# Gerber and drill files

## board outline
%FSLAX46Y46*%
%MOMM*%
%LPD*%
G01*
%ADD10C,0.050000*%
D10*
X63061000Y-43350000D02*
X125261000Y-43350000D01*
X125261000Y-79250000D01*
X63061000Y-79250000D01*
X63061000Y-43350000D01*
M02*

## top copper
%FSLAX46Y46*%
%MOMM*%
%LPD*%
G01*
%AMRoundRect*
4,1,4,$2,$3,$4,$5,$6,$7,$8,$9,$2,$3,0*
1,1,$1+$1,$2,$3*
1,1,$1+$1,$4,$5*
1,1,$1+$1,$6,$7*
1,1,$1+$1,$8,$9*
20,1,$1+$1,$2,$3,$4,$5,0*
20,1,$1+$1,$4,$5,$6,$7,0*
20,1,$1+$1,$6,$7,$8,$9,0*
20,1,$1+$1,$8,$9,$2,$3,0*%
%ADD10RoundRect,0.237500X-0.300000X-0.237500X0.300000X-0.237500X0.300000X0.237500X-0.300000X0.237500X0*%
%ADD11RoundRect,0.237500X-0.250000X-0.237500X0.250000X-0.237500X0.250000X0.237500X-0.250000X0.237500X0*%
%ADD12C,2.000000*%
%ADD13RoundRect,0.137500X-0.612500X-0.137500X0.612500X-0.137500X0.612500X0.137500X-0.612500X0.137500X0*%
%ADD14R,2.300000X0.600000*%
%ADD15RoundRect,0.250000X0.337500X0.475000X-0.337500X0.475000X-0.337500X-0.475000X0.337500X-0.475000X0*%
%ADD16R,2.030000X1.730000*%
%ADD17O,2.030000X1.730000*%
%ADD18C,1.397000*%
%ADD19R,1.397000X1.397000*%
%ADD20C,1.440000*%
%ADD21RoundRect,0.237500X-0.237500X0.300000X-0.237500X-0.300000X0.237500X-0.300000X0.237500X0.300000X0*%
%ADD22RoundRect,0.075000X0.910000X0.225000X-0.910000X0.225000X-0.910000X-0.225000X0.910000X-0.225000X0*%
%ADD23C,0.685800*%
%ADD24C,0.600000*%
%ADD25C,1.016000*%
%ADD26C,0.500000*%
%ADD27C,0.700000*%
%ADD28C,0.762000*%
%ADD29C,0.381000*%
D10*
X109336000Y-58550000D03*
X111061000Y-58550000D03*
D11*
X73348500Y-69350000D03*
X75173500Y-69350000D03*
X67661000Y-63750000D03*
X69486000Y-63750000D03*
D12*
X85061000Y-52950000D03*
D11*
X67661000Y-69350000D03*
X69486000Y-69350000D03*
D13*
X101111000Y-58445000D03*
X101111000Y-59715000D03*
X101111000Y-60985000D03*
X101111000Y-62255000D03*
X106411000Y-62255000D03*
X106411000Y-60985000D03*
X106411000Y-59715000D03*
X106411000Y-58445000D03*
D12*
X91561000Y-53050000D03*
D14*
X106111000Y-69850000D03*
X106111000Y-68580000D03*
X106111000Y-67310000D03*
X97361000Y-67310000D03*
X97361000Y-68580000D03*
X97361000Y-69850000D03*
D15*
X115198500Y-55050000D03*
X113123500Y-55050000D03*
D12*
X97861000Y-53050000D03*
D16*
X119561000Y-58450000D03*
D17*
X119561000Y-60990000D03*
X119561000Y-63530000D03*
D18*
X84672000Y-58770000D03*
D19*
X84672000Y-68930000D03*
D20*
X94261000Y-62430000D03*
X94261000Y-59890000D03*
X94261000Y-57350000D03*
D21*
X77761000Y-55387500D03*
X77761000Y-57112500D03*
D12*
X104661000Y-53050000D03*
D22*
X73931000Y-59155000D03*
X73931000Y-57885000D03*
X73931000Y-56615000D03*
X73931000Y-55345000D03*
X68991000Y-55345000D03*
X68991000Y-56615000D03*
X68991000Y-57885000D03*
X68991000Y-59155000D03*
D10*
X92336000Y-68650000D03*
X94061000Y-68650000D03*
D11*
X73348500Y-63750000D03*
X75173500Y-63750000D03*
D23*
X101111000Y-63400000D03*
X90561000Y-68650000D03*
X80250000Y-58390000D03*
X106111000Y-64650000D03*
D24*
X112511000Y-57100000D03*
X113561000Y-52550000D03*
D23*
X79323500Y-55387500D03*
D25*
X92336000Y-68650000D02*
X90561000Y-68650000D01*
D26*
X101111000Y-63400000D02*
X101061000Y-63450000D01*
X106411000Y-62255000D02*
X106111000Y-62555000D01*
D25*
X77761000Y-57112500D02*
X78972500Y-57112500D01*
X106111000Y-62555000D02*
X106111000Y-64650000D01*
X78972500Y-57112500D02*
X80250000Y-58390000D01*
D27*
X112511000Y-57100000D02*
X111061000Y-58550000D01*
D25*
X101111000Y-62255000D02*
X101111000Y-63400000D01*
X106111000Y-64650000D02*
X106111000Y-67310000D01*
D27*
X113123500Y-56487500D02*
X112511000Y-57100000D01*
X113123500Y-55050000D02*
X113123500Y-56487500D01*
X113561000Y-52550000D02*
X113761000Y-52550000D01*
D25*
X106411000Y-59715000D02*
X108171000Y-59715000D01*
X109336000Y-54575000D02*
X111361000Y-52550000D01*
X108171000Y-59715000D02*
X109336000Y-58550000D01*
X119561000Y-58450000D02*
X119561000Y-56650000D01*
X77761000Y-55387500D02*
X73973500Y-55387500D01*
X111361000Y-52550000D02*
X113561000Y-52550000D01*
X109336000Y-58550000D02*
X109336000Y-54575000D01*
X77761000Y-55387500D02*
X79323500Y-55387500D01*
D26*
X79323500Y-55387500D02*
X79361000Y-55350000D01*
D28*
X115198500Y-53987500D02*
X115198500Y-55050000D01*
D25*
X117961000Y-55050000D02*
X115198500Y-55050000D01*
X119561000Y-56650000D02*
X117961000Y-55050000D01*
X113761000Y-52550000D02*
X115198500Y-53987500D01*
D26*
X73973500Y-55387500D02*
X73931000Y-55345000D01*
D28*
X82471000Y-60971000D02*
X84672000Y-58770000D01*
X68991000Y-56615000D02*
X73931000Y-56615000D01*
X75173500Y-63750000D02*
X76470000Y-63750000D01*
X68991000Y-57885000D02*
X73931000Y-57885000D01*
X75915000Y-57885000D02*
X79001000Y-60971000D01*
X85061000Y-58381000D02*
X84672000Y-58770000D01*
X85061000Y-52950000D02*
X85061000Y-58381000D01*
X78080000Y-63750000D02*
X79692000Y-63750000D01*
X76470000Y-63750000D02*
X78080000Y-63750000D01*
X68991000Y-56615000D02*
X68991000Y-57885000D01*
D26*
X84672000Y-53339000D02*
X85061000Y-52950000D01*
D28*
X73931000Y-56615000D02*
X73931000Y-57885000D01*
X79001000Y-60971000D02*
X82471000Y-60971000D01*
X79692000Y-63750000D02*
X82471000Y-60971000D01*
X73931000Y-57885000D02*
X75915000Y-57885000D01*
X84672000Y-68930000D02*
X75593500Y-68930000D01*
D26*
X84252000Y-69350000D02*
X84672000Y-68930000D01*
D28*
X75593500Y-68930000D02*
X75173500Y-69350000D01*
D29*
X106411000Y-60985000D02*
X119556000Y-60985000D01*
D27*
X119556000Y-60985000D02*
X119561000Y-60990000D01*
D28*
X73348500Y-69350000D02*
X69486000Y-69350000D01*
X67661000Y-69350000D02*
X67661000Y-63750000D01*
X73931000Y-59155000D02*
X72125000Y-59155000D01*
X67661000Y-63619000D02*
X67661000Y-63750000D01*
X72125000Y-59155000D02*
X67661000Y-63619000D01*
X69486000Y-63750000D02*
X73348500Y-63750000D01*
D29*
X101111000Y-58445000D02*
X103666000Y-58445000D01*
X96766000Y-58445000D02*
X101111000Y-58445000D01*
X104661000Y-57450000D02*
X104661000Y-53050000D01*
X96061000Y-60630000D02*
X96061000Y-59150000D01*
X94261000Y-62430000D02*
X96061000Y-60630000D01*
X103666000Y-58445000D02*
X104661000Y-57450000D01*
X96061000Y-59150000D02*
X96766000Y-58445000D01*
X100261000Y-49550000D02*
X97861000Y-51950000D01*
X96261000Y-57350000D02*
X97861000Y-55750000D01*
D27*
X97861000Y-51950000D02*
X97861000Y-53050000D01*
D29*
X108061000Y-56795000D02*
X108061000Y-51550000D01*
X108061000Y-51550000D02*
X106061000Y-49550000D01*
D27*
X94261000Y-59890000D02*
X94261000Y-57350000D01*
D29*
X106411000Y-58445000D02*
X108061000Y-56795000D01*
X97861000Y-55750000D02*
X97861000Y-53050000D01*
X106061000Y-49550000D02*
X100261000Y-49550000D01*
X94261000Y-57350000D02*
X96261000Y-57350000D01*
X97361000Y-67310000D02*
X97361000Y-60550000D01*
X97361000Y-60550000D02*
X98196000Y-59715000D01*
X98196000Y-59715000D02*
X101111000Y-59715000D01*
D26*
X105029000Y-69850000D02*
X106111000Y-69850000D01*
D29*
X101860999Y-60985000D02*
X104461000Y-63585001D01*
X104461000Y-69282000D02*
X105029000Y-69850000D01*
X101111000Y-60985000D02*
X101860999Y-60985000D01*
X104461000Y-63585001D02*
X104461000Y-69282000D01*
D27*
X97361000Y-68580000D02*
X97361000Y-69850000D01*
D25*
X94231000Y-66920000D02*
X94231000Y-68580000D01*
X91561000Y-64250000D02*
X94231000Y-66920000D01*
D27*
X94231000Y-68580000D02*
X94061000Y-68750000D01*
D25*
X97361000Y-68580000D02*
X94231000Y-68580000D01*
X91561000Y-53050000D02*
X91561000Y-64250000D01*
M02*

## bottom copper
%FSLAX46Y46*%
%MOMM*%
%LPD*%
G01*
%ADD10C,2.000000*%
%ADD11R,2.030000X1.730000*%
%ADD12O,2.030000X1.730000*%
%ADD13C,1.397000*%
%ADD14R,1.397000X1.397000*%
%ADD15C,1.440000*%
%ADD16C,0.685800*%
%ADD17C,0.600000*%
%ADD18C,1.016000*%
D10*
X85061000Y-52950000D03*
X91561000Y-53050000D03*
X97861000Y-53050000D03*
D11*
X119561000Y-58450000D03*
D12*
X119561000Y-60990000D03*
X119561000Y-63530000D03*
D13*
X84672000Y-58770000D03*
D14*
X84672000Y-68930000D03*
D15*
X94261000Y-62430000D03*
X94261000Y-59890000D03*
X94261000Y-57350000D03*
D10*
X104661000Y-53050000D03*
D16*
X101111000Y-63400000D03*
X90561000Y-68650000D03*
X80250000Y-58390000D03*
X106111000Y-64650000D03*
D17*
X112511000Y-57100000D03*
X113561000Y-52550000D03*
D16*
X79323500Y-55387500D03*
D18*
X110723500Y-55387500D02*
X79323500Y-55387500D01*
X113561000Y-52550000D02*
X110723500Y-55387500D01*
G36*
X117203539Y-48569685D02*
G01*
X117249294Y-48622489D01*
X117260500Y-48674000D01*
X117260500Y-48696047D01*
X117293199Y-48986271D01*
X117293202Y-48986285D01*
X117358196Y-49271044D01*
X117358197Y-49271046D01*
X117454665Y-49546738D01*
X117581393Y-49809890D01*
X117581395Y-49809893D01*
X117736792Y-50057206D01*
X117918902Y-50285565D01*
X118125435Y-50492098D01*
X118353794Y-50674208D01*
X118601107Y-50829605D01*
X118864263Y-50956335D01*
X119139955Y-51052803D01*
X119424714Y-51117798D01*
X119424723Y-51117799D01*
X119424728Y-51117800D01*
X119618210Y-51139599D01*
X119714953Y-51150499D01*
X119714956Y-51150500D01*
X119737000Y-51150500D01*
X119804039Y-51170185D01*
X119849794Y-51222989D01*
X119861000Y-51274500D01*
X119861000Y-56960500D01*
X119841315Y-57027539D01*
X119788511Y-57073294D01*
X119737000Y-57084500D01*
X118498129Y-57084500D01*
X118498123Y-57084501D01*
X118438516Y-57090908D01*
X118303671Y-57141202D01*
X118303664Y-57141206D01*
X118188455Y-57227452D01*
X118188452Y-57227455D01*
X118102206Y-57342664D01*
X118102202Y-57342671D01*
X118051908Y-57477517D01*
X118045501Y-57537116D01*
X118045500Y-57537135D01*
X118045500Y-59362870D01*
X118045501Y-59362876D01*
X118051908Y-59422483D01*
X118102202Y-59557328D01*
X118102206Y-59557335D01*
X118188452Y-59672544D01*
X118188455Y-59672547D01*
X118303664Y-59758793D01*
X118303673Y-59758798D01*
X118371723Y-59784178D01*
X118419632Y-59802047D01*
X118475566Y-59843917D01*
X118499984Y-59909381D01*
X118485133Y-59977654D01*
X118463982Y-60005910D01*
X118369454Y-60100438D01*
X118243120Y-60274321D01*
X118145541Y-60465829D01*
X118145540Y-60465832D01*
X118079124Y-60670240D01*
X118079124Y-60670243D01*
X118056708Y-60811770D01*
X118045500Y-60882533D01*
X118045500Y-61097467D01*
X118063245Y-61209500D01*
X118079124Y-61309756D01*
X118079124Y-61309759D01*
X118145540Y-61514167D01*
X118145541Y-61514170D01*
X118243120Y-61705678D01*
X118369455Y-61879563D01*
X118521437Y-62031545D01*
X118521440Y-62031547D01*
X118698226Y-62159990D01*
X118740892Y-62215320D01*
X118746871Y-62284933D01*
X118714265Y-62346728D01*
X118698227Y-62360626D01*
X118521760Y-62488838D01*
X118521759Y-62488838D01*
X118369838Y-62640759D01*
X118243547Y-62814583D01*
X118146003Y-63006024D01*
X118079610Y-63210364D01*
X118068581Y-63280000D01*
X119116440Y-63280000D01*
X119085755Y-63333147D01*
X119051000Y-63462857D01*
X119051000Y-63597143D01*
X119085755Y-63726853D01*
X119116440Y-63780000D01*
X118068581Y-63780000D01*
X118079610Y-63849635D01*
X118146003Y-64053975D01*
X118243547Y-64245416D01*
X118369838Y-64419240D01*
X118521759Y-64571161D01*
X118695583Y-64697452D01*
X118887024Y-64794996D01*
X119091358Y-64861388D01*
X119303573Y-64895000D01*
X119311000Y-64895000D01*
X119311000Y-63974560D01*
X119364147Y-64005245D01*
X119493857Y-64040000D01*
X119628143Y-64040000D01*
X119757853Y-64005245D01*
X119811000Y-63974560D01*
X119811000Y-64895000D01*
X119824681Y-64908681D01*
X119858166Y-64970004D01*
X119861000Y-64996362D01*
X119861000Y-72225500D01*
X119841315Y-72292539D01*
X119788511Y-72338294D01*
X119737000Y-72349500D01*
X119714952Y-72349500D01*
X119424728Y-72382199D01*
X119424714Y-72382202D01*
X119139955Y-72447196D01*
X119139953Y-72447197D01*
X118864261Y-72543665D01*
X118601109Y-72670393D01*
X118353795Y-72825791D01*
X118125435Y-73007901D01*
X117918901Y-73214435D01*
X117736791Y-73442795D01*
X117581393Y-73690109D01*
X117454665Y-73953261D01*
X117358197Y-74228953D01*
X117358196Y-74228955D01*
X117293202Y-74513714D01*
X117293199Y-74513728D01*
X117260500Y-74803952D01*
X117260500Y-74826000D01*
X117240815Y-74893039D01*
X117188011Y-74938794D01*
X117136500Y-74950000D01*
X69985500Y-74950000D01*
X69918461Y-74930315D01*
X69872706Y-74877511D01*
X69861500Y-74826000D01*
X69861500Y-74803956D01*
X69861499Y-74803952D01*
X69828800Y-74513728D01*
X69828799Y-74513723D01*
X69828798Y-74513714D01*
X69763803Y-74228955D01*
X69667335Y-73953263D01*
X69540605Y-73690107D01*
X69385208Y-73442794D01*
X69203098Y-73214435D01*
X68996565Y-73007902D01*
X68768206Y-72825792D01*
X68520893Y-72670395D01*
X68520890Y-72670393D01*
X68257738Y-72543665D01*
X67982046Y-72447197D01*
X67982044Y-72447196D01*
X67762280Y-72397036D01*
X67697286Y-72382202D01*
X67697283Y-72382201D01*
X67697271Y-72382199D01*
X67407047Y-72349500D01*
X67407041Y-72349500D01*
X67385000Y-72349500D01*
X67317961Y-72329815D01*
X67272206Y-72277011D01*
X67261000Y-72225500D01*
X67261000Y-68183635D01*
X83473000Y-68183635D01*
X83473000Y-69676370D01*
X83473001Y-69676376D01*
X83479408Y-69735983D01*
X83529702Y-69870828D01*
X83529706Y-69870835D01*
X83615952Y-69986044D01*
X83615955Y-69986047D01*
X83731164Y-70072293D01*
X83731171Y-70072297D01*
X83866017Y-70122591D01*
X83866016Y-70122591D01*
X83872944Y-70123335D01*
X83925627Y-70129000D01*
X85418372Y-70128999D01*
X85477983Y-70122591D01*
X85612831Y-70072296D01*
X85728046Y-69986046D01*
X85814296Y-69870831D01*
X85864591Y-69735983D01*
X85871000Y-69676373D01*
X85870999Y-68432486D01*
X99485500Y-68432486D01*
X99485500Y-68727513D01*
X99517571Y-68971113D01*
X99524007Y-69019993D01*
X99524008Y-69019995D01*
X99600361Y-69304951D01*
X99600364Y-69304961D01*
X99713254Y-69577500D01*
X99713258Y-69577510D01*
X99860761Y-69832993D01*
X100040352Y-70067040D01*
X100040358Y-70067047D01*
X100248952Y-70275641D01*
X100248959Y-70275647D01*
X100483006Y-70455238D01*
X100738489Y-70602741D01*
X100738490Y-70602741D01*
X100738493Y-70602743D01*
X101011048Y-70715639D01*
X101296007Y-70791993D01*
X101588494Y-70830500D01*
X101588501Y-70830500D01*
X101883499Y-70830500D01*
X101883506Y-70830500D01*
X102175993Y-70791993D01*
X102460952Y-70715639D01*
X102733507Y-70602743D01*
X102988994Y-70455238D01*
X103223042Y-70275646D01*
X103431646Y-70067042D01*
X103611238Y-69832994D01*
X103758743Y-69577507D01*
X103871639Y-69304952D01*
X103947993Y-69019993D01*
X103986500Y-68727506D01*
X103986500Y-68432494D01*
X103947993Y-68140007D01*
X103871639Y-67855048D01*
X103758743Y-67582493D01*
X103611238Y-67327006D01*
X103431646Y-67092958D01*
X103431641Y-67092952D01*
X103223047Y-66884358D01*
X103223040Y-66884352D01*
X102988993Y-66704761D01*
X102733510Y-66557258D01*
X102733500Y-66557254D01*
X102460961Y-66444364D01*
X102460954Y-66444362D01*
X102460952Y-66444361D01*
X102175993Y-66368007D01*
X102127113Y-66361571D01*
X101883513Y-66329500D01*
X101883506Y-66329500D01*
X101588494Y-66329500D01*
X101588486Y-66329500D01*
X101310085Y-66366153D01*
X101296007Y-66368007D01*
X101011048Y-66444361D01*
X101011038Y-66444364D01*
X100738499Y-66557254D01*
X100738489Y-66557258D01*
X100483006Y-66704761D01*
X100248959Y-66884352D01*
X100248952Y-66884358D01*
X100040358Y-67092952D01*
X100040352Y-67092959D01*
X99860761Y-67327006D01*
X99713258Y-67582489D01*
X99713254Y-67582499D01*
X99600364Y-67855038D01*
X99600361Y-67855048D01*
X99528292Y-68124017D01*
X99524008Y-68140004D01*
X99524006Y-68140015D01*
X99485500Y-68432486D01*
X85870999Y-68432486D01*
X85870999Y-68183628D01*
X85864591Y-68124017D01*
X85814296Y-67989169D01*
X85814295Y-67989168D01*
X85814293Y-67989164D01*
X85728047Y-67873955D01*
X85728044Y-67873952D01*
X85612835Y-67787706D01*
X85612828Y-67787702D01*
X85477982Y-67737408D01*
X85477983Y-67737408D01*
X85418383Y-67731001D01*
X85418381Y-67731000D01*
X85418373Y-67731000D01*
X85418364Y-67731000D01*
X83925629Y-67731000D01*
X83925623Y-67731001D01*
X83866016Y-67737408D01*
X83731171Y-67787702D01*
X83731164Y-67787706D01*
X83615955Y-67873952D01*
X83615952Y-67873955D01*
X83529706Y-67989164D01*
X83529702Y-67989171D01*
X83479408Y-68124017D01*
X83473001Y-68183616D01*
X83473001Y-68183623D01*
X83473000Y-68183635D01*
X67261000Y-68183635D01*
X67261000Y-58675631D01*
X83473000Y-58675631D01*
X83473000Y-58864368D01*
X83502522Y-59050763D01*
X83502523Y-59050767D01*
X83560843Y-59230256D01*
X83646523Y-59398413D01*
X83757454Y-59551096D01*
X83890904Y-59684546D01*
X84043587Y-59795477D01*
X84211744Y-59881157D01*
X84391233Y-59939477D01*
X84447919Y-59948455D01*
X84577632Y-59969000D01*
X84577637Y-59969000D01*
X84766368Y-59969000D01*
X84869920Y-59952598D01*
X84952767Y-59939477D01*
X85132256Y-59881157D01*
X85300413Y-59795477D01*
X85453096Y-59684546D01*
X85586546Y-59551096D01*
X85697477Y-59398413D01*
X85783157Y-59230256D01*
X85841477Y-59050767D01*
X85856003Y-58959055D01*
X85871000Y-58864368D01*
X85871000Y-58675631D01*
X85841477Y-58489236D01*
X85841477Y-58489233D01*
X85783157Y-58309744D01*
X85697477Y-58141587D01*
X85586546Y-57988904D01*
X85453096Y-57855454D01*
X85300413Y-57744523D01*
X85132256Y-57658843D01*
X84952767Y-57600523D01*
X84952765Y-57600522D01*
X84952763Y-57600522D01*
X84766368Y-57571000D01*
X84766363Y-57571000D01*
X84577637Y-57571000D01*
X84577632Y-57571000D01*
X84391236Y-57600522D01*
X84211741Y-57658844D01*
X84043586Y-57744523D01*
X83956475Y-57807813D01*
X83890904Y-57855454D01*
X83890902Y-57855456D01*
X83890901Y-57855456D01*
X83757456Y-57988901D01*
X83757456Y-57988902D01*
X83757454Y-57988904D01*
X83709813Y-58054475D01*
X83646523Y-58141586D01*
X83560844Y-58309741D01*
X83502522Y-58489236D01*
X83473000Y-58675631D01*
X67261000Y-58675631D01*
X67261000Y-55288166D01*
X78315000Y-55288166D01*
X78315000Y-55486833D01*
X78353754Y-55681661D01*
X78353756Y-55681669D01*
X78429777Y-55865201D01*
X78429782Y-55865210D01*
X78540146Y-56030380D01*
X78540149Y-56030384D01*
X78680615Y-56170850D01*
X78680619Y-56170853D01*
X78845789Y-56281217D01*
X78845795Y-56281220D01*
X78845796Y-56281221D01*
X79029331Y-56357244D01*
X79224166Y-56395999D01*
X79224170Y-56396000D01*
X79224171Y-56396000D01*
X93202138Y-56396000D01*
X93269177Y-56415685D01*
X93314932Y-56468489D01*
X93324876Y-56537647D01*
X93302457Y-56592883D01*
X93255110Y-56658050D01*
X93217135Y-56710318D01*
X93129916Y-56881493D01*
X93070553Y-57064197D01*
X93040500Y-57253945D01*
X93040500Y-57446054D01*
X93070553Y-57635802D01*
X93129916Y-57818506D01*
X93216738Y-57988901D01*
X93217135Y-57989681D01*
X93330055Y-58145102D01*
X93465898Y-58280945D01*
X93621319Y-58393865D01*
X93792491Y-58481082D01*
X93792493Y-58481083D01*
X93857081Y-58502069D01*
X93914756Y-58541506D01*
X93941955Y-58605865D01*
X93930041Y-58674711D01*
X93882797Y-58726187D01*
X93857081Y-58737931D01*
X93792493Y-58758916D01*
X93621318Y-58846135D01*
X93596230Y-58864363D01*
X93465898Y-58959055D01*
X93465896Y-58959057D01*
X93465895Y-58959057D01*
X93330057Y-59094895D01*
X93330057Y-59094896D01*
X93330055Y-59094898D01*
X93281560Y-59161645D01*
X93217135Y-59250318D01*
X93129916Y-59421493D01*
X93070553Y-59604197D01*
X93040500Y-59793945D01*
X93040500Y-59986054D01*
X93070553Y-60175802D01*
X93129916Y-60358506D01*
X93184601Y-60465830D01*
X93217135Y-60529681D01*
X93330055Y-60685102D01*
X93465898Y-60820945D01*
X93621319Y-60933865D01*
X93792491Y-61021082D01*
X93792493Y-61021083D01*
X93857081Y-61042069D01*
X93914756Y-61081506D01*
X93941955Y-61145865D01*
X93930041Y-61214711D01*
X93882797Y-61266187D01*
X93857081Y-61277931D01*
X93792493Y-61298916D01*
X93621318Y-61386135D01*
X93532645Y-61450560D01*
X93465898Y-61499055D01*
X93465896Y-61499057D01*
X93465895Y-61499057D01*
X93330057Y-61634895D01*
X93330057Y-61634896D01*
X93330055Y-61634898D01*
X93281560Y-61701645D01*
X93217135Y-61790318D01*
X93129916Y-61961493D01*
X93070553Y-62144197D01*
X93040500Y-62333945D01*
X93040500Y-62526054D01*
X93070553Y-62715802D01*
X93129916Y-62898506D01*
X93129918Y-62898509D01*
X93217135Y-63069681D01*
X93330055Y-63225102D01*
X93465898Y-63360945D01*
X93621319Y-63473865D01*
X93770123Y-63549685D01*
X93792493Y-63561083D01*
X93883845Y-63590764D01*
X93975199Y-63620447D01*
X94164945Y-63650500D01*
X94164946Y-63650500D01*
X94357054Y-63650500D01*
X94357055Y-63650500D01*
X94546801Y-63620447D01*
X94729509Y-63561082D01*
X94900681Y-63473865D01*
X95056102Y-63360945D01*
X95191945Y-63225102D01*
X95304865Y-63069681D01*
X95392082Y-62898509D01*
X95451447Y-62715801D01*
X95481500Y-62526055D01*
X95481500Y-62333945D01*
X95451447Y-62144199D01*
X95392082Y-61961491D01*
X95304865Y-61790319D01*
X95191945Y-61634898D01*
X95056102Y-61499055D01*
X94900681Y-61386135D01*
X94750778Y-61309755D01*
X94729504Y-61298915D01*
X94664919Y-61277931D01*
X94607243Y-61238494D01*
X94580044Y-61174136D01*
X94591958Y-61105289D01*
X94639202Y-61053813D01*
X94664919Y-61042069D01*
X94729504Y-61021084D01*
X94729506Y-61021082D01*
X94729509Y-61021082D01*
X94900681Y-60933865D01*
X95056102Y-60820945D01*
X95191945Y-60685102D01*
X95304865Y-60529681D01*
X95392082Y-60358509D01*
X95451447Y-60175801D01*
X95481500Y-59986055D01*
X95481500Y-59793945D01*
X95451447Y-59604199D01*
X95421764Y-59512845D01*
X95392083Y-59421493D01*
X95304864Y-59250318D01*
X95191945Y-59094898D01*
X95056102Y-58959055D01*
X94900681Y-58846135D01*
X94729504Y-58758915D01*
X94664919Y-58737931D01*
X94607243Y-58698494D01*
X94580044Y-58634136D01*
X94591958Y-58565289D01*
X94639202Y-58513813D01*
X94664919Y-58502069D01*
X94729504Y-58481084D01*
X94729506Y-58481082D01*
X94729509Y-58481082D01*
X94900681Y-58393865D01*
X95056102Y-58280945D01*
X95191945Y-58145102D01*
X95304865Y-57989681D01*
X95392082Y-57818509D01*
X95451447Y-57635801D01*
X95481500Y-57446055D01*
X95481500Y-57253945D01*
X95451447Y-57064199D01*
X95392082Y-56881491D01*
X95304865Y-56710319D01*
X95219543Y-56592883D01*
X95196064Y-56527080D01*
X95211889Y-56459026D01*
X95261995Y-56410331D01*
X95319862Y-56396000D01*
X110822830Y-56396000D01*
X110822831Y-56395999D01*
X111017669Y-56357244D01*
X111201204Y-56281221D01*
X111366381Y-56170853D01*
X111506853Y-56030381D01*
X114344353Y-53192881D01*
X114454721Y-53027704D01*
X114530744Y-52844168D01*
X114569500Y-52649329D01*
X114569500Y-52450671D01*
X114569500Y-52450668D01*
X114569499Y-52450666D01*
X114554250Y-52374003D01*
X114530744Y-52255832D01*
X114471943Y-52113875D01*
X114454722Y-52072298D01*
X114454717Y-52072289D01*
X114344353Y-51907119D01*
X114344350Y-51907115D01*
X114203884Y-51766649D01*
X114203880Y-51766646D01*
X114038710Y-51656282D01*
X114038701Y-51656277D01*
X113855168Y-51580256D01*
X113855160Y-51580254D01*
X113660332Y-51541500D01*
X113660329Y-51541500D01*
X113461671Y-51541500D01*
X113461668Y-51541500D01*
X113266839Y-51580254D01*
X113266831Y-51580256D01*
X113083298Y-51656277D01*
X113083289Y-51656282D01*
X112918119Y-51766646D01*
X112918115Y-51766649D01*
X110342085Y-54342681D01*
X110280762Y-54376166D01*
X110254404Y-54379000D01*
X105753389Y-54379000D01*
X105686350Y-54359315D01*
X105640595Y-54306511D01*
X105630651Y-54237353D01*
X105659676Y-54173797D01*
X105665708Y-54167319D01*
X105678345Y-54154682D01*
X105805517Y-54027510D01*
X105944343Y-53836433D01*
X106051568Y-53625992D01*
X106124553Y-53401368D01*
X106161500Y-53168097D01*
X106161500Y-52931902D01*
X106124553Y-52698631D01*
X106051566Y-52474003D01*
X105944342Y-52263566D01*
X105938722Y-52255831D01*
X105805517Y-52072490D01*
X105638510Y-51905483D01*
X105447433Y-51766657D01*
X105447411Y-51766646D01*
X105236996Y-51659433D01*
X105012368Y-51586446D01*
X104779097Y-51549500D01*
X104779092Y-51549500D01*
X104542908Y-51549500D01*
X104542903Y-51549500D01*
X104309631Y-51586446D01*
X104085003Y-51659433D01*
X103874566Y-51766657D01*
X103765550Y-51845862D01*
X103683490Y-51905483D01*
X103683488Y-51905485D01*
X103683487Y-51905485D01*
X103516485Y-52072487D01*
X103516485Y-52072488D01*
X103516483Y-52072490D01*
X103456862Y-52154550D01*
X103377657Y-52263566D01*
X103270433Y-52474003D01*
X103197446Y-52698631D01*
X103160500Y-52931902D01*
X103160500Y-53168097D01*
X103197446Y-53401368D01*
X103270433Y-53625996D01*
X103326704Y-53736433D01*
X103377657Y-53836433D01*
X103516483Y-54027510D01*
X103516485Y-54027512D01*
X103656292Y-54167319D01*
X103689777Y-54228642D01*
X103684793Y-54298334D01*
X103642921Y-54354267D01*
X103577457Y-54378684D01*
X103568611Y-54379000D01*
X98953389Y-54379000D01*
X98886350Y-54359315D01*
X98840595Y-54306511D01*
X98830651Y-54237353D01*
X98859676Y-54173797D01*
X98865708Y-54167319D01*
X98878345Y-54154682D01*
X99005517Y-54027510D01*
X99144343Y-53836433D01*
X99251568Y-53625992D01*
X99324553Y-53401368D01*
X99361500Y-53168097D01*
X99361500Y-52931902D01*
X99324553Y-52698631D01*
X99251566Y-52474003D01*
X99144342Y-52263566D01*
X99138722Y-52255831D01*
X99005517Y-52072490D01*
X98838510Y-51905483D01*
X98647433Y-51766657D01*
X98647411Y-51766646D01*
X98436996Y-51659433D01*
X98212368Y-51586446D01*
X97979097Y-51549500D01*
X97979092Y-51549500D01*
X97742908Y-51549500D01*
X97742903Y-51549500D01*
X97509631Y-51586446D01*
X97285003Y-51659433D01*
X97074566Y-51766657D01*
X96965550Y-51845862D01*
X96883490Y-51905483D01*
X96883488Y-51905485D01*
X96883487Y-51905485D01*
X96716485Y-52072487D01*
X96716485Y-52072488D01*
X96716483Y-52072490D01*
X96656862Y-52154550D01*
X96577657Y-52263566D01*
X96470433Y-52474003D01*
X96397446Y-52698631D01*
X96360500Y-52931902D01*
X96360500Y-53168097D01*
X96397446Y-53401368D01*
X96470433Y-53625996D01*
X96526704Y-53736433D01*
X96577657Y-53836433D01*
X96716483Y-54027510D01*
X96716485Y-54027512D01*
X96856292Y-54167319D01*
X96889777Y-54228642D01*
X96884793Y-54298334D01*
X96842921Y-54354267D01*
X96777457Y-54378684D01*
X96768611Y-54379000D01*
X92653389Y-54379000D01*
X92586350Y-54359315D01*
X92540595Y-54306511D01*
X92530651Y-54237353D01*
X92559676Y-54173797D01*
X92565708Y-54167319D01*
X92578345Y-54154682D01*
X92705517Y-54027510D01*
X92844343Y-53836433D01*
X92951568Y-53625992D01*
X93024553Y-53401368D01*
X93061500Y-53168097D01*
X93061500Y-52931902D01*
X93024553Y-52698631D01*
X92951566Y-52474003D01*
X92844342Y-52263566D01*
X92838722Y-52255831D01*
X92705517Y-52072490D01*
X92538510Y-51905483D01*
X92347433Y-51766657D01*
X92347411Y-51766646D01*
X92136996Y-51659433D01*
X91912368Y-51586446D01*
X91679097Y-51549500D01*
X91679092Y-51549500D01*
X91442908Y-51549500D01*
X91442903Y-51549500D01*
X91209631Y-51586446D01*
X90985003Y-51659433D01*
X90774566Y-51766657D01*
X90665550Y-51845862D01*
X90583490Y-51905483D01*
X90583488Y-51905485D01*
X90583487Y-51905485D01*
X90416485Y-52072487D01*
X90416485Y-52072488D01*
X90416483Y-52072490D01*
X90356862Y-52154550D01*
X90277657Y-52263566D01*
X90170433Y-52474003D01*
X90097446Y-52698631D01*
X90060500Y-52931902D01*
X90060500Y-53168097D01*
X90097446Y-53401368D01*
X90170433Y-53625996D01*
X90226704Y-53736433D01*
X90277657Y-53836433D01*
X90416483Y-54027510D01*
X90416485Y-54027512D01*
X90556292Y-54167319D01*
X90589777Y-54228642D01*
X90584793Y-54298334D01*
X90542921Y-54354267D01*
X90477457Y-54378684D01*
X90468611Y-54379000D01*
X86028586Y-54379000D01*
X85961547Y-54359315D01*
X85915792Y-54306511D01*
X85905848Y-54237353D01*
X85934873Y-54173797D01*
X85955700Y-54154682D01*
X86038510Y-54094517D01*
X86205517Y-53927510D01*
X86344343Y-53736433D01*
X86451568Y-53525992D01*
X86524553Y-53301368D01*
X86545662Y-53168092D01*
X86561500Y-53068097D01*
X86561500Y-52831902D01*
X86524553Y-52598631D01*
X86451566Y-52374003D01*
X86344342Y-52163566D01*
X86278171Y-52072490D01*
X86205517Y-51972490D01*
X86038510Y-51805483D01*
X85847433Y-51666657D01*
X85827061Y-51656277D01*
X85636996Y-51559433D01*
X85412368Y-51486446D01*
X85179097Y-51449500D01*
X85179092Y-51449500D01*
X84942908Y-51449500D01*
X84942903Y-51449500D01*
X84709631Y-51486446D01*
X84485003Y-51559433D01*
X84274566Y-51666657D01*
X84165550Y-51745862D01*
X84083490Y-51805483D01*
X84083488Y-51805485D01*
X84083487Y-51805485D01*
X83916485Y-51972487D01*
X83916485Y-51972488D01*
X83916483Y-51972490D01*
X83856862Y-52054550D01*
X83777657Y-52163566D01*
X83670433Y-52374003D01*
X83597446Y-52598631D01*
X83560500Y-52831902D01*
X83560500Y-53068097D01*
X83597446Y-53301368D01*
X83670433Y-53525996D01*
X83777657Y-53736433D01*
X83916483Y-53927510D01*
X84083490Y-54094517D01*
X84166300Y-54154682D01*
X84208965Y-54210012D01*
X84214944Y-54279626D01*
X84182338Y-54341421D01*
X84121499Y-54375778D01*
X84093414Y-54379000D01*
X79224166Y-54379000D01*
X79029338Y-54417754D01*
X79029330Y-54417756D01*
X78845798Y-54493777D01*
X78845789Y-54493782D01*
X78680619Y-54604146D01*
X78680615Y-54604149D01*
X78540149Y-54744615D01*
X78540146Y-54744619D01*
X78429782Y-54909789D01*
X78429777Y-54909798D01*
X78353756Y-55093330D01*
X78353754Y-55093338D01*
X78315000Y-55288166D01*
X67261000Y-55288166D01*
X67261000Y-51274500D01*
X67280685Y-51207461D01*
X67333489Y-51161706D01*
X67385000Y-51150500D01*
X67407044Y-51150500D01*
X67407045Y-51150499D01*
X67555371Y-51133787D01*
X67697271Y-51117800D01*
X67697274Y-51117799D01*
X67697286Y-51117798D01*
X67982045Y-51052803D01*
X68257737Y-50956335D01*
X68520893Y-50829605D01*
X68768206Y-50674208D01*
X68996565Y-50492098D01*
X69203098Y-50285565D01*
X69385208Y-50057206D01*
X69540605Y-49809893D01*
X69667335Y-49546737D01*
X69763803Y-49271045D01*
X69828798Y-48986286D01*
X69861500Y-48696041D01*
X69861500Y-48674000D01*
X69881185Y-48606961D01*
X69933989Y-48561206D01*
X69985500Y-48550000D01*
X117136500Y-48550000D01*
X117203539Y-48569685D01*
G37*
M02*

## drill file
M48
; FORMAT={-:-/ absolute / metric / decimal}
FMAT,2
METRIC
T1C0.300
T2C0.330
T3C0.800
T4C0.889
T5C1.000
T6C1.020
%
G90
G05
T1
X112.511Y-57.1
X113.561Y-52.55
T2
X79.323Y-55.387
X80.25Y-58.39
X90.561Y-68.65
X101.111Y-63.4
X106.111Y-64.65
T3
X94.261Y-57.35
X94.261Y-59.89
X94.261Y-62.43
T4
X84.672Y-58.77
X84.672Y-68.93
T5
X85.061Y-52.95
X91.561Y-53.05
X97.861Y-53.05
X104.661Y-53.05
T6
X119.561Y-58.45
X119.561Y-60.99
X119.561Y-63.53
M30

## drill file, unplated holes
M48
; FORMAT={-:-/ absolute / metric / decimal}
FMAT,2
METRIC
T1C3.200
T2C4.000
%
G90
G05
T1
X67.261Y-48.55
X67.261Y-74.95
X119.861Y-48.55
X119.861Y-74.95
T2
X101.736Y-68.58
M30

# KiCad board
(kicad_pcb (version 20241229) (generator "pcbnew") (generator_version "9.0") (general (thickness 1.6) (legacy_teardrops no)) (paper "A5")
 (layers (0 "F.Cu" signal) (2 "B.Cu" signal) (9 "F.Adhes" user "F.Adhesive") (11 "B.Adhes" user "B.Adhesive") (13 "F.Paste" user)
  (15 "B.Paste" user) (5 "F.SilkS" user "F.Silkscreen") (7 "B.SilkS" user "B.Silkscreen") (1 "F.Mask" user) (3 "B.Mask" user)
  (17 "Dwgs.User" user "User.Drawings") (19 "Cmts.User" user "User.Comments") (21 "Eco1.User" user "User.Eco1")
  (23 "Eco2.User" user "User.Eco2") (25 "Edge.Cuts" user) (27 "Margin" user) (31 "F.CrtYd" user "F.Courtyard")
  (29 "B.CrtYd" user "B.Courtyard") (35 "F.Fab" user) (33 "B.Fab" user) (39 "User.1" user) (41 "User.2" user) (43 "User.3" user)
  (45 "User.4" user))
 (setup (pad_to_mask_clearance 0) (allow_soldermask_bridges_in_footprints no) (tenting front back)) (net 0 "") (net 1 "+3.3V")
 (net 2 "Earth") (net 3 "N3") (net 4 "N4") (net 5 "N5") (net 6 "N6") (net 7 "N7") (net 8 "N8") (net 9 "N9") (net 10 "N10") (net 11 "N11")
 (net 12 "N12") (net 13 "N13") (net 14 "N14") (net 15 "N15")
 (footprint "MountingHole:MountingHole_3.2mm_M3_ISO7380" (layer "F.Cu") (at 67.261 48.55)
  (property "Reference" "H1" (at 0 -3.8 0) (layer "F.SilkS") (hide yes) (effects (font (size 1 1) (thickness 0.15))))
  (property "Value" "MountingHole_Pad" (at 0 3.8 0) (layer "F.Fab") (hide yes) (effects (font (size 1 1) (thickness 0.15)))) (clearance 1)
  (pad "" np_thru_hole circle (at 0 0) (size 3.2 3.2) (drill 3.2) (layers "*.Cu" "*.Mask")))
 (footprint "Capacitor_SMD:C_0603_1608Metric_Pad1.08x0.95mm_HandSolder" (layer "F.Cu") (at 110.1985 58.55)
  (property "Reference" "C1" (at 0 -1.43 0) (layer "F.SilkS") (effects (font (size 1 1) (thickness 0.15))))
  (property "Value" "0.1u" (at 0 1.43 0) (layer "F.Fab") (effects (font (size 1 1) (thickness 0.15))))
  (pad "1" smd roundrect (at -0.8625 0) (size 1.075 0.95) (layers "F.Cu" "F.Mask" "F.Paste") (roundrect_rratio 0.25) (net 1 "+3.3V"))
  (pad "2" smd roundrect (at 0.8625 0) (size 1.075 0.95) (layers "F.Cu" "F.Mask" "F.Paste") (roundrect_rratio 0.25) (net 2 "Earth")))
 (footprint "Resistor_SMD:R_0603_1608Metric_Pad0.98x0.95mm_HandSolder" (layer "F.Cu") (at 74.261 69.35)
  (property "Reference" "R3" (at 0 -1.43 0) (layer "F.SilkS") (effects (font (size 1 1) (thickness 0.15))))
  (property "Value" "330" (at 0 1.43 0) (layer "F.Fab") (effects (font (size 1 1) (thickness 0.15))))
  (pad "1" smd roundrect (at -0.9125 0) (size 0.975 0.95) (layers "F.Cu" "F.Mask" "F.Paste") (roundrect_rratio 0.25) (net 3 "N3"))
  (pad "2" smd roundrect (at 0.9125 0) (size 0.975 0.95) (layers "F.Cu" "F.Mask" "F.Paste") (roundrect_rratio 0.25) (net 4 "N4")))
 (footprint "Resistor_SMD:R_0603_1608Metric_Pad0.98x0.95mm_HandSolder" (layer "F.Cu") (at 68.5735 63.75)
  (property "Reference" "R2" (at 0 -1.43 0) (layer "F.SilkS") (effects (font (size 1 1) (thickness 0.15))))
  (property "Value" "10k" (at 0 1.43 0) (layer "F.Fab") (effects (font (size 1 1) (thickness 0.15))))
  (pad "1" smd roundrect (at -0.9125 0) (size 0.975 0.95) (layers "F.Cu" "F.Mask" "F.Paste") (roundrect_rratio 0.25) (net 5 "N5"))
  (pad "2" smd roundrect (at 0.9125 0) (size 0.975 0.95) (layers "F.Cu" "F.Mask" "F.Paste") (roundrect_rratio 0.25) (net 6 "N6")))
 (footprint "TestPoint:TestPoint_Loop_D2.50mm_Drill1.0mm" (layer "F.Cu") (at 85.061 52.95 180)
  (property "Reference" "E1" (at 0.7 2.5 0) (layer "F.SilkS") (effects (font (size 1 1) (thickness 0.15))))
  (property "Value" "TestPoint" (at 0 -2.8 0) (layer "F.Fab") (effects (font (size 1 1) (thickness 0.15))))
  (pad "1" thru_hole circle (at 0 0 180) (size 2 2) (drill 1) (layers "*.Cu" "*.Mask") (remove_unused_layers no) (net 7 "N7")))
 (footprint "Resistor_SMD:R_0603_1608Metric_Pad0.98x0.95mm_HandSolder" (layer "F.Cu") (at 68.5735 69.35)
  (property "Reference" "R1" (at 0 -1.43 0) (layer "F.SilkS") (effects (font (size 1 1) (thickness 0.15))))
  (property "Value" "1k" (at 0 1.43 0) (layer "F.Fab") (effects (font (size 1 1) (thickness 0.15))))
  (pad "1" smd roundrect (at -0.9125 0) (size 0.975 0.95) (layers "F.Cu" "F.Mask" "F.Paste") (roundrect_rratio 0.25) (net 5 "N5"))
  (pad "2" smd roundrect (at 0.9125 0) (size 0.975 0.95) (layers "F.Cu" "F.Mask" "F.Paste") (roundrect_rratio 0.25) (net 3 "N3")))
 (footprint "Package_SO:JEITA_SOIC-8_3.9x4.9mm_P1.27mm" (layer "F.Cu") (at 103.761 60.35)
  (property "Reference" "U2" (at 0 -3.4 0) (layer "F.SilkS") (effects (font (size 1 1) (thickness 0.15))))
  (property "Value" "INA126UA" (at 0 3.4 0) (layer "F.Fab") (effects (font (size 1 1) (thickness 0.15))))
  (pad "1" smd roundrect (at -2.65 -1.905) (size 1.5 0.55) (layers "F.Cu" "F.Mask" "F.Paste") (roundrect_rratio 0.25) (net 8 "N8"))
  (pad "2" smd roundrect (at -2.65 -0.635) (size 1.5 0.55) (layers "F.Cu" "F.Mask" "F.Paste") (roundrect_rratio 0.25) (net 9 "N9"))
  (pad "3" smd roundrect (at -2.65 0.635) (size 1.5 0.55) (layers "F.Cu" "F.Mask" "F.Paste") (roundrect_rratio 0.25) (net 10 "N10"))
  (pad "4" smd roundrect (at -2.65 1.905) (size 1.5 0.55) (layers "F.Cu" "F.Mask" "F.Paste") (roundrect_rratio 0.25) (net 2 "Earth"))
  (pad "5" smd roundrect (at 2.65 1.905) (size 1.5 0.55) (layers "F.Cu" "F.Mask" "F.Paste") (roundrect_rratio 0.25) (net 2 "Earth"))
  (pad "6" smd roundrect (at 2.65 0.635) (size 1.5 0.55) (layers "F.Cu" "F.Mask" "F.Paste") (roundrect_rratio 0.25) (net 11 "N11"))
  (pad "7" smd roundrect (at 2.65 -0.635) (size 1.5 0.55) (layers "F.Cu" "F.Mask" "F.Paste") (roundrect_rratio 0.25) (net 1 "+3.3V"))
  (pad "8" smd roundrect (at 2.65 -1.905) (size 1.5 0.55) (layers "F.Cu" "F.Mask" "F.Paste") (roundrect_rratio 0.25) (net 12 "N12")))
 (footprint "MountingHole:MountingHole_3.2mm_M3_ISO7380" (layer "F.Cu") (at 119.861 48.55)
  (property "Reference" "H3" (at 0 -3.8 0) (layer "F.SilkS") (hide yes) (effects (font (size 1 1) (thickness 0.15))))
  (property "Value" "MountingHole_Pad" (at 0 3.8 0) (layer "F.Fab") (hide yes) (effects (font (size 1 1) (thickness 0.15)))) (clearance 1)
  (pad "" np_thru_hole circle (at 0 0) (size 3.2 3.2) (drill 3.2) (layers "*.Cu" "*.Mask")))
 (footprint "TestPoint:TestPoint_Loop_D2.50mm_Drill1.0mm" (layer "F.Cu") (at 91.561 53.05 180)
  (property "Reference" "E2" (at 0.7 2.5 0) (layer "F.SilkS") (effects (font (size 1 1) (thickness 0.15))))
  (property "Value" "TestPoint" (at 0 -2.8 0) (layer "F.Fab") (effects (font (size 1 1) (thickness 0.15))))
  (pad "1" thru_hole circle (at 0 0 180) (size 2 2) (drill 1) (layers "*.Cu" "*.Mask") (remove_unused_layers no) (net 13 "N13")))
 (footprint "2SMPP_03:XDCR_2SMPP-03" (layer "F.Cu") (at 101.736 68.58 180)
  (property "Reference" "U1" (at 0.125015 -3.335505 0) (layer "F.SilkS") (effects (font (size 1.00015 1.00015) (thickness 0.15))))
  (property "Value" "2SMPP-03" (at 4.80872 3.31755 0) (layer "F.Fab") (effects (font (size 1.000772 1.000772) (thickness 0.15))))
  (pad "" np_thru_hole circle (at 0 0 180) (size 4 4) (drill 4) (layers "*.Cu" "*.Mask") (clearance 0.05))
  (pad "1" smd rect (at -4.375 -1.27 180) (size 2.3 0.6) (layers "F.Cu" "F.Mask" "F.Paste") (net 10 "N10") (solder_mask_margin 0.102))
  (pad "2" smd rect (at -4.375 0 180) (size 2.3 0.6) (layers "F.Cu" "F.Mask" "F.Paste") (solder_mask_margin 0.102))
  (pad "3" smd rect (at -4.375 1.27 180) (size 2.3 0.6) (layers "F.Cu" "F.Mask" "F.Paste") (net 2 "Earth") (solder_mask_margin 0.102))
  (pad "4" smd rect (at 4.375 1.27 180) (size 2.3 0.6) (layers "F.Cu" "F.Mask" "F.Paste") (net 9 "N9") (solder_mask_margin 0.102))
  (pad "5" smd rect (at 4.375 0 180) (size 2.3 0.6) (layers "F.Cu" "F.Mask" "F.Paste") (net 13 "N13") (solder_mask_margin 0.102))
  (pad "6" smd rect (at 4.375 -1.27 180) (size 2.3 0.6) (layers "F.Cu" "F.Mask" "F.Paste") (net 13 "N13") (solder_mask_margin 0.102)))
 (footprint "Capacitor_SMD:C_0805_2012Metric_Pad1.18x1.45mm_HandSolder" (layer "F.Cu") (at 114.161 55.05 180)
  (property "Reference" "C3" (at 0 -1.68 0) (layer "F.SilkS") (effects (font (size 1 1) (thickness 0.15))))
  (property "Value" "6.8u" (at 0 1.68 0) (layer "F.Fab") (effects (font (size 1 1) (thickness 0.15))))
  (pad "1" smd roundrect (at -1.0375 0 180) (size 1.175 1.45) (layers "F.Cu" "F.Mask" "F.Paste") (roundrect_rratio 0.212766) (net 1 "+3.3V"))
  (pad "2" smd roundrect (at 1.0375 0 180) (size 1.175 1.45) (layers "F.Cu" "F.Mask" "F.Paste") (roundrect_rratio 0.212766) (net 2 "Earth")))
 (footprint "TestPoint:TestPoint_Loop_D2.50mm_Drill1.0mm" (layer "F.Cu") (at 97.861 53.05 180)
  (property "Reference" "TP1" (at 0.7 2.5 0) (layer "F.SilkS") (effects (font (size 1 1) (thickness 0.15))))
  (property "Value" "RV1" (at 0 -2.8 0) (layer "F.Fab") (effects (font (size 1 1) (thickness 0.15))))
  (pad "1" thru_hole circle (at 0 0 180) (size 2 2) (drill 1) (layers "*.Cu" "*.Mask") (remove_unused_layers no) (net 12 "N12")))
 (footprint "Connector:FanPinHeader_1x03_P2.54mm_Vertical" (layer "F.Cu") (at 119.561 58.45 -90)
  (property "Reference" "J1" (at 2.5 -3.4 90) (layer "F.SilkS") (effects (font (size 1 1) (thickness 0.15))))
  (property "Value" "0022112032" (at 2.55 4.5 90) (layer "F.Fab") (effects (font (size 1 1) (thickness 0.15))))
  (pad "1" thru_hole rect (at 0 0) (size 2.03 1.73) (drill 1.02) (layers "*.Cu" "*.Mask") (remove_unused_layers no) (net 1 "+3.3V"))
  (pad "2" thru_hole oval (at 2.54 0) (size 2.03 1.73) (drill 1.02) (layers "*.Cu" "*.Mask") (remove_unused_layers no) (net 11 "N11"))
  (pad "3" thru_hole oval (at 5.08 0) (size 2.03 1.73) (drill 1.02) (layers "*.Cu" "*.Mask") (remove_unused_layers no) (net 2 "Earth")))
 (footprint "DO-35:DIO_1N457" (layer "F.Cu") (at 84.672 68.93 -90)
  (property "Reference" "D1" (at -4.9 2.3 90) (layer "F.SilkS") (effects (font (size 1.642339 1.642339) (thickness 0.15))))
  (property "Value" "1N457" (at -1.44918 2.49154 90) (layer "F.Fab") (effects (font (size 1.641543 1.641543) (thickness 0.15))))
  (pad "1" thru_hole circle (at -10.16 0 270) (size 1.397 1.397) (drill 0.889) (layers "*.Cu" "*.Mask") (remove_unused_layers no)
   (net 7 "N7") (solder_mask_margin 0.102))
  (pad "2" thru_hole rect (at 0 0 270) (size 1.397 1.397) (drill 0.889) (layers "*.Cu" "*.Mask") (remove_unused_layers no) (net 4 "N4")
   (solder_mask_margin 0.102)))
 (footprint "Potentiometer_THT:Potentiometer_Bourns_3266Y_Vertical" (layer "F.Cu") (at 94.261 62.43 -90)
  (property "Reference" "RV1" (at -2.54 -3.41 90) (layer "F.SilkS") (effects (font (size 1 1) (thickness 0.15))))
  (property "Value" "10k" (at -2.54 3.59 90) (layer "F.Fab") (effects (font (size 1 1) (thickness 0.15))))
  (pad "1" thru_hole circle (at 0 0 270) (size 1.44 1.44) (drill 0.8) (layers "*.Cu" "*.Mask") (remove_unused_layers no) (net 8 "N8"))
  (pad "2" thru_hole circle (at -2.54 0 270) (size 1.44 1.44) (drill 0.8) (layers "*.Cu" "*.Mask") (remove_unused_layers no) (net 12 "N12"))
  (pad "3" thru_hole circle (at -5.08 0 270) (size 1.44 1.44) (drill 0.8) (layers "*.Cu" "*.Mask") (remove_unused_layers no) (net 12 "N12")))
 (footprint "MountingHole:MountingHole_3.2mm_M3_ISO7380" (layer "F.Cu") (at 67.261 74.95)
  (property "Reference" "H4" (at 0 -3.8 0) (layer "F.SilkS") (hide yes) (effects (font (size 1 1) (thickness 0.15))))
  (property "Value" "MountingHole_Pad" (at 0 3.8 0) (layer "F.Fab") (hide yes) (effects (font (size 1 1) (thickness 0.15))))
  (pad "" np_thru_hole circle (at 0 0) (size 3.2 3.2) (drill 3.2) (layers "*.Cu" "*.Mask") (clearance 1)))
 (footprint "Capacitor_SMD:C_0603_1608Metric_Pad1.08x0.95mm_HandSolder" (layer "F.Cu") (at 77.761 56.25 -90)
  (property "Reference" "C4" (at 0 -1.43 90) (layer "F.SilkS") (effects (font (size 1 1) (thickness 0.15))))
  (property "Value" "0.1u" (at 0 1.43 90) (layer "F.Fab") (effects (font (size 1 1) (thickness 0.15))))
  (pad "1" smd roundrect (at -0.8625 0 270) (size 1.075 0.95) (layers "F.Cu" "F.Mask" "F.Paste") (roundrect_rratio 0.25) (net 1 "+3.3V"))
  (pad "2" smd roundrect (at 0.8625 0 270) (size 1.075 0.95) (layers "F.Cu" "F.Mask" "F.Paste") (roundrect_rratio 0.25) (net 2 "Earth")))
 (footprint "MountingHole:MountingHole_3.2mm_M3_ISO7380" (layer "F.Cu") (at 119.861 74.95)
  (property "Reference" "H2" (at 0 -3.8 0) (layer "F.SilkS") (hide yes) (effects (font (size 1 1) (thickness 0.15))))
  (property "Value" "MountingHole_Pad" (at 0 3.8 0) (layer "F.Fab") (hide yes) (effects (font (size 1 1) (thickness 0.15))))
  (pad "" np_thru_hole circle (at 0 0) (size 3.2 3.2) (drill 3.2) (layers "*.Cu" "*.Mask") (clearance 1)))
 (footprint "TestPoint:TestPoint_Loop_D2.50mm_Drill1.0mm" (layer "F.Cu") (at 104.661 53.05 180)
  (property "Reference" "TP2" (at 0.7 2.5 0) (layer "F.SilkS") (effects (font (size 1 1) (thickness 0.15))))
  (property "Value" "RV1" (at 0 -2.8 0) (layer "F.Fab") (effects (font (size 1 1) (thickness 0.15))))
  (pad "1" thru_hole circle (at 0 0 180) (size 2 2) (drill 1) (layers "*.Cu" "*.Mask") (remove_unused_layers no) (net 8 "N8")))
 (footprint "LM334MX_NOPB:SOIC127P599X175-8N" (layer "F.Cu") (at 71.461 57.25 180)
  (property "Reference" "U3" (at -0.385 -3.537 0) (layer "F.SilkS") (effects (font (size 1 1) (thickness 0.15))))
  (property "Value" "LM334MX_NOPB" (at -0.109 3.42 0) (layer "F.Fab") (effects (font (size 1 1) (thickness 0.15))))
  (pad "1" smd roundrect (at -2.47 -1.905 180) (size 1.97 0.6) (layers "F.Cu" "F.Mask" "F.Paste") (roundrect_rratio 0.125) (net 5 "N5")
   (solder_mask_margin 0.102))
  (pad "2" smd roundrect (at -2.47 -0.635 180) (size 1.97 0.6) (layers "F.Cu" "F.Mask" "F.Paste") (roundrect_rratio 0.125) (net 7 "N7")
   (solder_mask_margin 0.102))
  (pad "3" smd roundrect (at -2.47 0.635 180) (size 1.97 0.6) (layers "F.Cu" "F.Mask" "F.Paste") (roundrect_rratio 0.125) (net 7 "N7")
   (solder_mask_margin 0.102))
  (pad "4" smd roundrect (at -2.47 1.905 180) (size 1.97 0.6) (layers "F.Cu" "F.Mask" "F.Paste") (roundrect_rratio 0.125) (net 1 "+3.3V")
   (solder_mask_margin 0.102))
  (pad "5" smd roundrect (at 2.47 1.905 180) (size 1.97 0.6) (layers "F.Cu" "F.Mask" "F.Paste") (roundrect_rratio 0.125) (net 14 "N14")
   (solder_mask_margin 0.102))
  (pad "6" smd roundrect (at 2.47 0.635 180) (size 1.97 0.6) (layers "F.Cu" "F.Mask" "F.Paste") (roundrect_rratio 0.125) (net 7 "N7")
   (solder_mask_margin 0.102))
  (pad "7" smd roundrect (at 2.47 -0.635 180) (size 1.97 0.6) (layers "F.Cu" "F.Mask" "F.Paste") (roundrect_rratio 0.125) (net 7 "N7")
   (solder_mask_margin 0.102))
  (pad "8" smd roundrect (at 2.47 -1.905 180) (size 1.97 0.6) (layers "F.Cu" "F.Mask" "F.Paste") (roundrect_rratio 0.125) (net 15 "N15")
   (solder_mask_margin 0.102)))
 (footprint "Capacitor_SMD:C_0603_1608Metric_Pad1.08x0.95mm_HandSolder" (layer "F.Cu") (at 93.1985 68.65)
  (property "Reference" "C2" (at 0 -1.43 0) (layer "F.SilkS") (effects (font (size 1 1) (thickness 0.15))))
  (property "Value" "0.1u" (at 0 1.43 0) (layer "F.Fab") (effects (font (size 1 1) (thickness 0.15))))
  (pad "1" smd roundrect (at -0.8625 0) (size 1.075 0.95) (layers "F.Cu" "F.Mask" "F.Paste") (roundrect_rratio 0.25) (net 2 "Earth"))
  (pad "2" smd roundrect (at 0.8625 0) (size 1.075 0.95) (layers "F.Cu" "F.Mask" "F.Paste") (roundrect_rratio 0.25) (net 13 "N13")))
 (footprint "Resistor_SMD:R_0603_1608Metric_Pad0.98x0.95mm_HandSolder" (layer "F.Cu") (at 74.261 63.75)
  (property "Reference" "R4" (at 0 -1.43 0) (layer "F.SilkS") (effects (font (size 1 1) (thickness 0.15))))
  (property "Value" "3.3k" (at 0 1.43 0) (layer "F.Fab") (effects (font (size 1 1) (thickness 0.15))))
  (pad "1" smd roundrect (at -0.9125 0) (size 0.975 0.95) (layers "F.Cu" "F.Mask" "F.Paste") (roundrect_rratio 0.25) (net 6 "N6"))
  (pad "2" smd roundrect (at 0.9125 0) (size 0.975 0.95) (layers "F.Cu" "F.Mask" "F.Paste") (roundrect_rratio 0.25) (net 7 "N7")))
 (gr_rect (start 63.061 43.35) (end 125.261 79.25) (stroke (width 0.05) (type default)) (fill no) (layer "Edge.Cuts"))
 (segment (start 92.336 68.65) (end 90.561 68.65) (width 1.016) (layer "F.Cu") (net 2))
 (segment (start 101.111 63.4) (end 101.061 63.45) (width 0.5) (layer "F.Cu") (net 2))
 (segment (start 106.411 62.255) (end 106.111 62.555) (width 0.5) (layer "F.Cu") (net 2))
 (segment (start 77.761 57.1125) (end 78.9725 57.1125) (width 1.016) (layer "F.Cu") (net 2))
 (segment (start 106.111 62.555) (end 106.111 64.65) (width 1.016) (layer "F.Cu") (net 2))
 (segment (start 78.9725 57.1125) (end 80.25 58.39) (width 1.016) (layer "F.Cu") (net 2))
 (segment (start 112.511 57.1) (end 111.061 58.55) (width 0.7) (layer "F.Cu") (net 2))
 (segment (start 101.111 62.255) (end 101.111 63.4) (width 1.016) (layer "F.Cu") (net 2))
 (segment (start 106.111 64.65) (end 106.111 67.31) (width 1.016) (layer "F.Cu") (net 2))
 (segment (start 113.1235 56.4875) (end 112.511 57.1) (width 0.7) (layer "F.Cu") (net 2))
 (segment (start 113.1235 55.05) (end 113.1235 56.4875) (width 0.7) (layer "F.Cu") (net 2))
 (via (at 101.111 63.4) (size 0.6858) (drill 0.3302) (layers "F.Cu" "B.Cu") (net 2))
 (via (at 90.561 68.65) (size 0.6858) (drill 0.3302) (layers "F.Cu" "B.Cu") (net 2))
 (via (at 80.25 58.39) (size 0.6858) (drill 0.3302) (layers "F.Cu" "B.Cu") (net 2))
 (via (at 106.111 64.65) (size 0.6858) (drill 0.3302) (layers "F.Cu" "B.Cu") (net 2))
 (via (at 112.511 57.1) (size 0.6) (drill 0.3) (layers "F.Cu" "B.Cu") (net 2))
 (segment (start 113.561 52.55) (end 113.761 52.55) (width 0.7) (layer "F.Cu") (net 1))
 (segment (start 106.411 59.715) (end 108.171 59.715) (width 1.016) (layer "F.Cu") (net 1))
 (segment (start 109.336 54.575) (end 111.361 52.55) (width 1.016) (layer "F.Cu") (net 1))
 (segment (start 108.171 59.715) (end 109.336 58.55) (width 1.016) (layer "F.Cu") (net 1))
 (segment (start 119.561 58.45) (end 119.561 56.65) (width 1.016) (layer "F.Cu") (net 1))
 (segment (start 77.761 55.3875) (end 73.9735 55.3875) (width 1.016) (layer "F.Cu") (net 1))
 (segment (start 111.361 52.55) (end 113.561 52.55) (width 1.016) (layer "F.Cu") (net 1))
 (segment (start 109.336 58.55) (end 109.336 54.575) (width 1.016) (layer "F.Cu") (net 1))
 (segment (start 77.761 55.3875) (end 79.3235 55.3875) (width 1.016) (layer "F.Cu") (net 1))
 (segment (start 79.3235 55.3875) (end 79.361 55.35) (width 0.5) (layer "F.Cu") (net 1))
 (segment (start 115.1985 53.9875) (end 115.1985 55.05) (width 0.762) (layer "F.Cu") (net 1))
 (segment (start 117.961 55.05) (end 115.1985 55.05) (width 1.016) (layer "F.Cu") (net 1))
 (segment (start 119.561 56.65) (end 117.961 55.05) (width 1.016) (layer "F.Cu") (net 1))
 (segment (start 113.761 52.55) (end 115.1985 53.9875) (width 1.016) (layer "F.Cu") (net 1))
 (segment (start 73.9735 55.3875) (end 73.931 55.345) (width 0.5) (layer "F.Cu") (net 1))
 (via (at 113.561 52.55) (size 0.6) (drill 0.3) (layers "F.Cu" "B.Cu") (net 1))
 (via (at 79.3235 55.3875) (size 0.6858) (drill 0.3302) (layers "F.Cu" "B.Cu") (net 1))
 (segment (start 110.7235 55.3875) (end 79.3235 55.3875) (width 1.016) (layer "B.Cu") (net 1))
 (segment (start 113.561 52.55) (end 110.7235 55.3875) (width 1.016) (layer "B.Cu") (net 1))
 (segment (start 82.471 60.971) (end 84.672 58.77) (width 0.762) (layer "F.Cu") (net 7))
 (segment (start 68.991 56.615) (end 73.931 56.615) (width 0.762) (layer "F.Cu") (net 7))
 (segment (start 75.1735 63.75) (end 76.47 63.75) (width 0.762) (layer "F.Cu") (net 7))
 (segment (start 68.991 57.885) (end 73.931 57.885) (width 0.762) (layer "F.Cu") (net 7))
 (segment (start 75.915 57.885) (end 79.001 60.971) (width 0.762) (layer "F.Cu") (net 7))
 (segment (start 85.061 58.381) (end 84.672 58.77) (width 0.762) (layer "F.Cu") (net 7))
 (segment (start 85.061 52.95) (end 85.061 58.381) (width 0.762) (layer "F.Cu") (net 7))
 (segment (start 78.08 63.75) (end 79.692 63.75) (width 0.762) (layer "F.Cu") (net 7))
 (segment (start 76.47 63.75) (end 78.08 63.75) (width 0.762) (layer "F.Cu") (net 7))
 (segment (start 68.991 56.615) (end 68.991 57.885) (width 0.762) (layer "F.Cu") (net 7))
 (segment (start 84.672 53.339) (end 85.061 52.95) (width 0.5) (layer "F.Cu") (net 7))
 (segment (start 73.931 56.615) (end 73.931 57.885) (width 0.762) (layer "F.Cu") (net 7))
 (segment (start 79.001 60.971) (end 82.471 60.971) (width 0.762) (layer "F.Cu") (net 7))
 (segment (start 79.692 63.75) (end 82.471 60.971) (width 0.762) (layer "F.Cu") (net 7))
 (segment (start 73.931 57.885) (end 75.915 57.885) (width 0.762) (layer "F.Cu") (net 7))
 (segment (start 84.672 68.93) (end 75.5935 68.93) (width 0.762) (layer "F.Cu") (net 4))
 (segment (start 84.252 69.35) (end 84.672 68.93) (width 0.5) (layer "F.Cu") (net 4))
 (segment (start 75.5935 68.93) (end 75.1735 69.35) (width 0.762) (layer "F.Cu") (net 4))
 (segment (start 106.411 60.985) (end 119.556 60.985) (width 0.381) (layer "F.Cu") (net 11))
 (segment (start 119.556 60.985) (end 119.561 60.99) (width 0.7) (layer "F.Cu") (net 11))
 (segment (start 73.3485 69.35) (end 69.486 69.35) (width 0.762) (layer "F.Cu") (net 3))
 (segment (start 67.661 69.35) (end 67.661 63.75) (width 0.762) (layer "F.Cu") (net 5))
 (segment (start 73.931 59.155) (end 72.125 59.155) (width 0.762) (layer "F.Cu") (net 5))
 (segment (start 67.661 63.619) (end 67.661 63.75) (width 0.762) (layer "F.Cu") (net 5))
 (segment (start 72.125 59.155) (end 67.661 63.619) (width 0.762) (layer "F.Cu") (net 5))
 (segment (start 69.486 63.75) (end 73.3485 63.75) (width 0.762) (layer "F.Cu") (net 6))
 (segment (start 101.111 58.445) (end 103.666 58.445) (width 0.381) (layer "F.Cu") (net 8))
 (segment (start 96.766 58.445) (end 101.111 58.445) (width 0.381) (layer "F.Cu") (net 8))
 (segment (start 104.661 57.45) (end 104.661 53.05) (width 0.381) (layer "F.Cu") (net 8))
 (segment (start 96.061 60.63) (end 96.061 59.15) (width 0.381) (layer "F.Cu") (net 8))
 (segment (start 94.261 62.43) (end 96.061 60.63) (width 0.381) (layer "F.Cu") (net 8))
 (segment (start 103.666 58.445) (end 104.661 57.45) (width 0.381) (layer "F.Cu") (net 8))
 (segment (start 96.061 59.15) (end 96.766 58.445) (width 0.381) (layer "F.Cu") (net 8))
 (segment (start 100.261 49.55) (end 97.861 51.95) (width 0.381) (layer "F.Cu") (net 12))
 (segment (start 96.261 57.35) (end 97.861 55.75) (width 0.381) (layer "F.Cu") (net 12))
 (segment (start 97.861 51.95) (end 97.861 53.05) (width 0.7) (layer "F.Cu") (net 12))
 (segment (start 108.061 56.795) (end 108.061 51.55) (width 0.381) (layer "F.Cu") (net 12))
 (segment (start 108.061 51.55) (end 106.061 49.55) (width 0.381) (layer "F.Cu") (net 12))
 (segment (start 94.261 59.89) (end 94.261 57.35) (width 0.7) (layer "F.Cu") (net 12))
 (segment (start 106.411 58.445) (end 108.061 56.795) (width 0.381) (layer "F.Cu") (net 12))
 (segment (start 97.861 55.75) (end 97.861 53.05) (width 0.381) (layer "F.Cu") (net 12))
 (segment (start 106.061 49.55) (end 100.261 49.55) (width 0.381) (layer "F.Cu") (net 12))
 (segment (start 94.261 57.35) (end 96.261 57.35) (width 0.381) (layer "F.Cu") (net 12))
 (segment (start 97.361 67.31) (end 97.361 60.55) (width 0.381) (layer "F.Cu") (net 9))
 (segment (start 97.361 60.55) (end 98.196 59.715) (width 0.381) (layer "F.Cu") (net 9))
 (segment (start 98.196 59.715) (end 101.111 59.715) (width 0.381) (layer "F.Cu") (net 9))
 (segment (start 105.029 69.85) (end 106.111 69.85) (width 0.5) (layer "F.Cu") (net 10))
 (segment (start 101.860999 60.985) (end 104.461 63.585001) (width 0.381) (layer "F.Cu") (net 10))
 (segment (start 104.461 69.282) (end 105.029 69.85) (width 0.381) (layer "F.Cu") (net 10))
 (segment (start 101.111 60.985) (end 101.860999 60.985) (width 0.381) (layer "F.Cu") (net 10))
 (segment (start 104.461 63.585001) (end 104.461 69.282) (width 0.381) (layer "F.Cu") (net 10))
 (segment (start 97.361 68.58) (end 97.361 69.85) (width 0.7) (layer "F.Cu") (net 13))
 (segment (start 94.231 66.92) (end 94.231 68.58) (width 1.016) (layer "F.Cu") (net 13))
 (segment (start 91.561 64.25) (end 94.231 66.92) (width 1.016) (layer "F.Cu") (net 13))
 (segment (start 94.231 68.58) (end 94.061 68.75) (width 0.7) (layer "F.Cu") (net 13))
 (segment (start 97.361 68.58) (end 94.231 68.58) (width 1.016) (layer "F.Cu") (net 13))
 (segment (start 91.561 53.05) (end 91.561 64.25) (width 1.016) (layer "F.Cu") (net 13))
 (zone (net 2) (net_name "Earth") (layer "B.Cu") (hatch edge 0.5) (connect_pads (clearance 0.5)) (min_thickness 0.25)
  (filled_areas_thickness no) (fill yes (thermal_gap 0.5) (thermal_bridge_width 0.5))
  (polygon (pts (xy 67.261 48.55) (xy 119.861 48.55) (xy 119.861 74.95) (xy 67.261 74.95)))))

